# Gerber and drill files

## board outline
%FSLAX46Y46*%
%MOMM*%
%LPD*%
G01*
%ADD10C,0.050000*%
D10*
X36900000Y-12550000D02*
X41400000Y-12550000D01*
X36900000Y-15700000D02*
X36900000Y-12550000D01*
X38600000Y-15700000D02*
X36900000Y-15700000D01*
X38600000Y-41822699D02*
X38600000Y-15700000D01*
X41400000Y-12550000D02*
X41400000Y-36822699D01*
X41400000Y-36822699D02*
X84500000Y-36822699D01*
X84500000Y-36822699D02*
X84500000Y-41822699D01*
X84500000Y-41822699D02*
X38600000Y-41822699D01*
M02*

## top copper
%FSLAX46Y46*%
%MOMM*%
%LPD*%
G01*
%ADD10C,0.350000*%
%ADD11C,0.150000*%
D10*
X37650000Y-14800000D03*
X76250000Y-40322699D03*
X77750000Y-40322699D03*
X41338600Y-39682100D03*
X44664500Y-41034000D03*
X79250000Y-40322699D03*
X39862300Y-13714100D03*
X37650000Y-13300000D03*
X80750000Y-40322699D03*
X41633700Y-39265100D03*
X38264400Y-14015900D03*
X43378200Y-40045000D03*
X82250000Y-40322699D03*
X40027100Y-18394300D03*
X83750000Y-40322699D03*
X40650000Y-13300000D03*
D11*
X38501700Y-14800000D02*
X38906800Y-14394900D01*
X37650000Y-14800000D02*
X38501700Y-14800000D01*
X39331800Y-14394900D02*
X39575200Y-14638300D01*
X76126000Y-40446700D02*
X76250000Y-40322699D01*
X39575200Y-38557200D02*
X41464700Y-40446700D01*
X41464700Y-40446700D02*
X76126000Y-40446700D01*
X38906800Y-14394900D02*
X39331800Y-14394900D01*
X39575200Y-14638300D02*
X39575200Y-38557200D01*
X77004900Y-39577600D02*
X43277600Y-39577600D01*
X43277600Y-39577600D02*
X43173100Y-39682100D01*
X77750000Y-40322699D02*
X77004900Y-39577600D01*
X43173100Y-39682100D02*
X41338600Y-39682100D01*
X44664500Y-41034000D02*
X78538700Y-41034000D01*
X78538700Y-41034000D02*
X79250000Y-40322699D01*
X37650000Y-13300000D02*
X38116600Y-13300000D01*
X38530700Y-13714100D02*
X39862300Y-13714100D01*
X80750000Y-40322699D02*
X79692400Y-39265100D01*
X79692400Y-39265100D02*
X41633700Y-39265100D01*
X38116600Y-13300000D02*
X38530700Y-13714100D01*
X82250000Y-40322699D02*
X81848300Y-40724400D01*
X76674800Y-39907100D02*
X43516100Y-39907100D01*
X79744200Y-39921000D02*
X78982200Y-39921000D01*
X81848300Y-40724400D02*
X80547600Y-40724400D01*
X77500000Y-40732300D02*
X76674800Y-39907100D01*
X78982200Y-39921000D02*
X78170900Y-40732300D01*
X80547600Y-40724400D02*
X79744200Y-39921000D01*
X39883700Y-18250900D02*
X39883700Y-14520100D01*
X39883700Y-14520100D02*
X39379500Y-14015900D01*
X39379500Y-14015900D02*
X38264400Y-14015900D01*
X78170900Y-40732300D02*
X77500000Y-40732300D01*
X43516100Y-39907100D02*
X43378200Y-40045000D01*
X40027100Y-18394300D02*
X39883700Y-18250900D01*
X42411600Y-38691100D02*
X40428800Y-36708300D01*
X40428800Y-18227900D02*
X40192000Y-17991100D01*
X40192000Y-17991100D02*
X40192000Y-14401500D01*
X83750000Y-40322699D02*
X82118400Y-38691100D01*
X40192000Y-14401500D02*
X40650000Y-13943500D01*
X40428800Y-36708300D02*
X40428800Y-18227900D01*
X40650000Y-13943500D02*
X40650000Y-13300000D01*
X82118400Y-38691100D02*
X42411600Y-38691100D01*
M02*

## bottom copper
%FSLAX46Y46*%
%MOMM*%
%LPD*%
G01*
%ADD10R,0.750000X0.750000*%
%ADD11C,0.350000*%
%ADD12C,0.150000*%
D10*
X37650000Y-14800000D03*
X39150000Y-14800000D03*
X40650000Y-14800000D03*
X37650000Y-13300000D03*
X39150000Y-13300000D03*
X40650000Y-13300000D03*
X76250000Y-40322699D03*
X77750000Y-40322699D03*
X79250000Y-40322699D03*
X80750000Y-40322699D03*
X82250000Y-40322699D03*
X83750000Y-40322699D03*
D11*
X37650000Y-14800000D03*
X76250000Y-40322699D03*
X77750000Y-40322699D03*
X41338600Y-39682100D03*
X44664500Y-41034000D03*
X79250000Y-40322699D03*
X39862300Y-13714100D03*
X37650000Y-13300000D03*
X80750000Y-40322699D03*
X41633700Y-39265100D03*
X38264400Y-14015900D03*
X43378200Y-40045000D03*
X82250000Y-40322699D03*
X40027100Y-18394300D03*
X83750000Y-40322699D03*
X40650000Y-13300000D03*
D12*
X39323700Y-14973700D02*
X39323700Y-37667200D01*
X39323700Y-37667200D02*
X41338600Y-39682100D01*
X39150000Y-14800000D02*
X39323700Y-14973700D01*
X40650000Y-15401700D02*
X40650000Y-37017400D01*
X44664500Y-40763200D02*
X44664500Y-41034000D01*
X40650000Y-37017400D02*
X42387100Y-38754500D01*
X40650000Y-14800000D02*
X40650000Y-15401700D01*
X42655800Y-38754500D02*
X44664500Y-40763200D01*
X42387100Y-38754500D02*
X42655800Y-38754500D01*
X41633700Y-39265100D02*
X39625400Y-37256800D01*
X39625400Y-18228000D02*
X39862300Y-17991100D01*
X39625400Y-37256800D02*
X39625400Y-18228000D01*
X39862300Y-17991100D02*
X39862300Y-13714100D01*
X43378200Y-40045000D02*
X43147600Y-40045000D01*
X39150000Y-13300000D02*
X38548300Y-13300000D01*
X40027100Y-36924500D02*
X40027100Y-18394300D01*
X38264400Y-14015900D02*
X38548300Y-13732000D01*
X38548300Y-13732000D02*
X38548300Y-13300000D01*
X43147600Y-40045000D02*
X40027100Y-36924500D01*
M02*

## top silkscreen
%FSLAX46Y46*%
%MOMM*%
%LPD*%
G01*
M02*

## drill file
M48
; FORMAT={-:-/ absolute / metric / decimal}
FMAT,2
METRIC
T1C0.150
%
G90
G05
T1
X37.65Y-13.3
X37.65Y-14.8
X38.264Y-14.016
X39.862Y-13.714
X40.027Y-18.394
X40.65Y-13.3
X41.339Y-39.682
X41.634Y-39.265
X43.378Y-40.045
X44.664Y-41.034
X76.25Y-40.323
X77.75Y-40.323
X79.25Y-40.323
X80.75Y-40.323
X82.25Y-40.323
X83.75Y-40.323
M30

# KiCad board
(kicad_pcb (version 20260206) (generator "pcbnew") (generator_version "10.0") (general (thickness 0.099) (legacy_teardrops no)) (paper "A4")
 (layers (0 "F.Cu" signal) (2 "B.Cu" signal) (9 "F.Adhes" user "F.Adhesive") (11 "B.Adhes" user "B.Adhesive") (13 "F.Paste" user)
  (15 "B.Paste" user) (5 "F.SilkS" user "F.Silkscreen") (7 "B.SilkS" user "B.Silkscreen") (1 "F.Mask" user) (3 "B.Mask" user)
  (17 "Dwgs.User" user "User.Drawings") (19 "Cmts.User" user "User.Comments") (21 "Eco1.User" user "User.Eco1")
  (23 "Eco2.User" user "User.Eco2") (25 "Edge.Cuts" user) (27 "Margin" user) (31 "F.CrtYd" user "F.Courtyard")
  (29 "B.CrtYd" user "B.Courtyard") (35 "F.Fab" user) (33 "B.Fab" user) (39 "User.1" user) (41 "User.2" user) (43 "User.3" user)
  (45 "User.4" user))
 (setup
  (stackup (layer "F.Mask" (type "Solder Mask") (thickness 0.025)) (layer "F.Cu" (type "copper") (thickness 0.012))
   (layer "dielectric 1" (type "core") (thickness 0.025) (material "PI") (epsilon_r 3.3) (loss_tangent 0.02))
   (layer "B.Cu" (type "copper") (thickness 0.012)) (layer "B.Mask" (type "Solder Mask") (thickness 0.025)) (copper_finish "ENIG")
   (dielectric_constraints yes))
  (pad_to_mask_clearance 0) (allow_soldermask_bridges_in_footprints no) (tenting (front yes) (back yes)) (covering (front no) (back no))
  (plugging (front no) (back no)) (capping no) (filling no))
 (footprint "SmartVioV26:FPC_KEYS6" (layer "F.Cu") (at 0 0)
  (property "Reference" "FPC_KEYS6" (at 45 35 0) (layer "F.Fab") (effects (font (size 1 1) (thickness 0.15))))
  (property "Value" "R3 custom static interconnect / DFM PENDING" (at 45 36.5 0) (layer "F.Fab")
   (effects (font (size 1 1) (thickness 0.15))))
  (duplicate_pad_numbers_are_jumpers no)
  (pad "S1" smd rect (at 37.65 14.8) (size 0.75 0.75) (layers "B.Cu" "B.Mask") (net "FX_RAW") (solder_mask_margin 0.1))
  (pad "S2" smd rect (at 39.15 14.8) (size 0.75 0.75) (layers "B.Cu" "B.Mask") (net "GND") (solder_mask_margin 0.1))
  (pad "S3" smd rect (at 40.65 14.8) (size 0.75 0.75) (layers "B.Cu" "B.Mask") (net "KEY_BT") (solder_mask_margin 0.1))
  (pad "S4" smd rect (at 37.65 13.3) (size 0.75 0.75) (layers "B.Cu" "B.Mask") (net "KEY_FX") (solder_mask_margin 0.1))
  (pad "S5" smd rect (at 39.15 13.3) (size 0.75 0.75) (layers "B.Cu" "B.Mask") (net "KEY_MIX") (solder_mask_margin 0.1))
  (pad "S6" smd rect (at 40.65 13.3) (size 0.75 0.75) (layers "B.Cu" "B.Mask") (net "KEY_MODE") (solder_mask_margin 0.1))
  (pad "T1" smd rect (at 76.25 40.322699) (size 0.75 0.75) (layers "B.Cu" "B.Mask") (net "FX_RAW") (solder_mask_margin 0.1))
  (pad "T2" smd rect (at 77.75 40.322699) (size 0.75 0.75) (layers "B.Cu" "B.Mask") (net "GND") (solder_mask_margin 0.1))
  (pad "T3" smd rect (at 79.25 40.322699) (size 0.75 0.75) (layers "B.Cu" "B.Mask") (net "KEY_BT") (solder_mask_margin 0.1))
  (pad "T4" smd rect (at 80.75 40.322699) (size 0.75 0.75) (layers "B.Cu" "B.Mask") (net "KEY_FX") (solder_mask_margin 0.1))
  (pad "T5" smd rect (at 82.25 40.322699) (size 0.75 0.75) (layers "B.Cu" "B.Mask") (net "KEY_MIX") (solder_mask_margin 0.1))
  (pad "T6" smd rect (at 83.75 40.322699) (size 0.75 0.75) (layers "B.Cu" "B.Mask") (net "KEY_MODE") (solder_mask_margin 0.1)))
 (gr_line (start 36.9 12.55) (end 41.4 12.55) (stroke (width 0.05) (type default)) (layer "Edge.Cuts"))
 (gr_line (start 36.9 15.7) (end 36.9 12.55) (stroke (width 0.05) (type default)) (layer "Edge.Cuts"))
 (gr_line (start 38.6 15.7) (end 36.9 15.7) (stroke (width 0.05) (type default)) (layer "Edge.Cuts"))
 (gr_line (start 38.6 41.822699) (end 38.6 15.7) (stroke (width 0.05) (type default)) (layer "Edge.Cuts"))
 (gr_line (start 41.4 12.55) (end 41.4 36.822699) (stroke (width 0.05) (type default)) (layer "Edge.Cuts"))
 (gr_line (start 41.4 36.822699) (end 84.5 36.822699) (stroke (width 0.05) (type default)) (layer "Edge.Cuts"))
 (gr_line (start 84.5 36.822699) (end 84.5 41.822699) (stroke (width 0.05) (type default)) (layer "Edge.Cuts"))
 (gr_line (start 84.5 41.822699) (end 38.6 41.822699) (stroke (width 0.05) (type default)) (layer "Edge.Cuts"))
 (segment (start 38.5017 14.8) (end 38.9068 14.3949) (width 0.15) (layer "F.Cu") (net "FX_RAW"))
 (segment (start 37.65 14.8) (end 38.5017 14.8) (width 0.15) (layer "F.Cu") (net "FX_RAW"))
 (segment (start 39.3318 14.3949) (end 39.5752 14.6383) (width 0.15) (layer "F.Cu") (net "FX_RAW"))
 (segment (start 76.126 40.4467) (end 76.25 40.322699) (width 0.15) (layer "F.Cu") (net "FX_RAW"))
 (segment (start 39.5752 38.5572) (end 41.4647 40.4467) (width 0.15) (layer "F.Cu") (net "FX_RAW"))
 (segment (start 41.4647 40.4467) (end 76.126 40.4467) (width 0.15) (layer "F.Cu") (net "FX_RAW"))
 (segment (start 38.9068 14.3949) (end 39.3318 14.3949) (width 0.15) (layer "F.Cu") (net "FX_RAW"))
 (segment (start 39.5752 14.6383) (end 39.5752 38.5572) (width 0.15) (layer "F.Cu") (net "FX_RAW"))
 (via (at 37.65 14.8) (size 0.35) (drill 0.15) (layers "F.Cu" "B.Cu") (locked yes) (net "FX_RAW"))
 (via (at 76.25 40.322699) (size 0.35) (drill 0.15) (layers "F.Cu" "B.Cu") (locked yes) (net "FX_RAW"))
 (segment (start 77.0049 39.5776) (end 43.2776 39.5776) (width 0.15) (layer "F.Cu") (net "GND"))
 (segment (start 43.2776 39.5776) (end 43.1731 39.6821) (width 0.15) (layer "F.Cu") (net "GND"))
 (segment (start 77.75 40.322699) (end 77.0049 39.5776) (width 0.15) (layer "F.Cu") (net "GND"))
 (segment (start 43.1731 39.6821) (end 41.3386 39.6821) (width 0.15) (layer "F.Cu") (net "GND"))
 (via (at 77.75 40.322699) (size 0.35) (drill 0.15) (layers "F.Cu" "B.Cu") (locked yes) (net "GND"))
 (via (at 41.3386 39.6821) (size 0.35) (drill 0.15) (layers "F.Cu" "B.Cu") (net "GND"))
 (segment (start 39.3237 14.9737) (end 39.3237 37.6672) (width 0.15) (layer "B.Cu") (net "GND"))
 (segment (start 39.3237 37.6672) (end 41.3386 39.6821) (width 0.15) (layer "B.Cu") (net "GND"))
 (segment (start 39.15 14.8) (end 39.3237 14.9737) (width 0.15) (layer "B.Cu") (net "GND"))
 (segment (start 44.6645 41.034) (end 78.5387 41.034) (width 0.15) (layer "F.Cu") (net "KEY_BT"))
 (segment (start 78.5387 41.034) (end 79.25 40.322699) (width 0.15) (layer "F.Cu") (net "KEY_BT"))
 (via (at 44.6645 41.034) (size 0.35) (drill 0.15) (layers "F.Cu" "B.Cu") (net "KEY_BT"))
 (via (at 79.25 40.322699) (size 0.35) (drill 0.15) (layers "F.Cu" "B.Cu") (locked yes) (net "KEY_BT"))
 (segment (start 40.65 15.4017) (end 40.65 37.0174) (width 0.15) (layer "B.Cu") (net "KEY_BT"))
 (segment (start 44.6645 40.7632) (end 44.6645 41.034) (width 0.15) (layer "B.Cu") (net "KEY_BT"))
 (segment (start 40.65 37.0174) (end 42.3871 38.7545) (width 0.15) (layer "B.Cu") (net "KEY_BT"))
 (segment (start 40.65 14.8) (end 40.65 15.4017) (width 0.15) (layer "B.Cu") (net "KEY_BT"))
 (segment (start 42.6558 38.7545) (end 44.6645 40.7632) (width 0.15) (layer "B.Cu") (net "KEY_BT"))
 (segment (start 42.3871 38.7545) (end 42.6558 38.7545) (width 0.15) (layer "B.Cu") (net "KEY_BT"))
 (segment (start 37.65 13.3) (end 38.1166 13.3) (width 0.15) (layer "F.Cu") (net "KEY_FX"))
 (segment (start 38.5307 13.7141) (end 39.8623 13.7141) (width 0.15) (layer "F.Cu") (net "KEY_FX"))
 (segment (start 80.75 40.322699) (end 79.6924 39.2651) (width 0.15) (layer "F.Cu") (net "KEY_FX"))
 (segment (start 79.6924 39.2651) (end 41.6337 39.2651) (width 0.15) (layer "F.Cu") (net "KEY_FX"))
 (segment (start 38.1166 13.3) (end 38.5307 13.7141) (width 0.15) (layer "F.Cu") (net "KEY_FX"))
 (via (at 39.8623 13.7141) (size 0.35) (drill 0.15) (layers "F.Cu" "B.Cu") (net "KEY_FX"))
 (via (at 37.65 13.3) (size 0.35) (drill 0.15) (layers "F.Cu" "B.Cu") (locked yes) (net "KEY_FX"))
 (via (at 80.75 40.322699) (size 0.35) (drill 0.15) (layers "F.Cu" "B.Cu") (locked yes) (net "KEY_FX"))
 (via (at 41.6337 39.2651) (size 0.35) (drill 0.15) (layers "F.Cu" "B.Cu") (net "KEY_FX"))
 (segment (start 41.6337 39.2651) (end 39.6254 37.2568) (width 0.15) (layer "B.Cu") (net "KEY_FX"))
 (segment (start 39.6254 18.228) (end 39.8623 17.9911) (width 0.15) (layer "B.Cu") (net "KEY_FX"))
 (segment (start 39.6254 37.2568) (end 39.6254 18.228) (width 0.15) (layer "B.Cu") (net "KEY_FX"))
 (segment (start 39.8623 17.9911) (end 39.8623 13.7141) (width 0.15) (layer "B.Cu") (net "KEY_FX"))
 (segment (start 82.25 40.322699) (end 81.8483 40.7244) (width 0.15) (layer "F.Cu") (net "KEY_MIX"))
 (segment (start 76.6748 39.9071) (end 43.5161 39.9071) (width 0.15) (layer "F.Cu") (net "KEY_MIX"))
 (segment (start 79.7442 39.921) (end 78.9822 39.921) (width 0.15) (layer "F.Cu") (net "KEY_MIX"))
 (segment (start 81.8483 40.7244) (end 80.5476 40.7244) (width 0.15) (layer "F.Cu") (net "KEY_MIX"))
 (segment (start 77.5 40.7323) (end 76.6748 39.9071) (width 0.15) (layer "F.Cu") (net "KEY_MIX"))
 (segment (start 78.9822 39.921) (end 78.1709 40.7323) (width 0.15) (layer "F.Cu") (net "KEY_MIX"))
 (segment (start 80.5476 40.7244) (end 79.7442 39.921) (width 0.15) (layer "F.Cu") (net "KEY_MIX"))
 (segment (start 39.8837 18.2509) (end 39.8837 14.5201) (width 0.15) (layer "F.Cu") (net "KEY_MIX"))
 (segment (start 39.8837 14.5201) (end 39.3795 14.0159) (width 0.15) (layer "F.Cu") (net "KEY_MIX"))
 (segment (start 39.3795 14.0159) (end 38.2644 14.0159) (width 0.15) (layer "F.Cu") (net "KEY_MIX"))
 (segment (start 78.1709 40.7323) (end 77.5 40.7323) (width 0.15) (layer "F.Cu") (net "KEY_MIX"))
 (segment (start 43.5161 39.9071) (end 43.3782 40.045) (width 0.15) (layer "F.Cu") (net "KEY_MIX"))
 (segment (start 40.0271 18.3943) (end 39.8837 18.2509) (width 0.15) (layer "F.Cu") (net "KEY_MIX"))
 (via (at 38.2644 14.0159) (size 0.35) (drill 0.15) (layers "F.Cu" "B.Cu") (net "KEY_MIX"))
 (via (at 43.3782 40.045) (size 0.35) (drill 0.15) (layers "F.Cu" "B.Cu") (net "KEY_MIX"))
 (via (at 82.25 40.322699) (size 0.35) (drill 0.15) (layers "F.Cu" "B.Cu") (locked yes) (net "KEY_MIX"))
 (via (at 40.0271 18.3943) (size 0.35) (drill 0.15) (layers "F.Cu" "B.Cu") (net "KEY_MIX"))
 (segment (start 43.3782 40.045) (end 43.1476 40.045) (width 0.15) (layer "B.Cu") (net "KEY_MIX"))
 (segment (start 39.15 13.3) (end 38.5483 13.3) (width 0.15) (layer "B.Cu") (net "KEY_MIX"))
 (segment (start 40.0271 36.9245) (end 40.0271 18.3943) (width 0.15) (layer "B.Cu") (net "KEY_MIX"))
 (segment (start 38.2644 14.0159) (end 38.5483 13.732) (width 0.15) (layer "B.Cu") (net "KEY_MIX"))
 (segment (start 38.5483 13.732) (end 38.5483 13.3) (width 0.15) (layer "B.Cu") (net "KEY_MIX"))
 (segment (start 43.1476 40.045) (end 40.0271 36.9245) (width 0.15) (layer "B.Cu") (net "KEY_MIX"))
 (segment (start 42.4116 38.6911) (end 40.4288 36.7083) (width 0.15) (layer "F.Cu") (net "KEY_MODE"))
 (segment (start 40.4288 18.2279) (end 40.192 17.9911) (width 0.15) (layer "F.Cu") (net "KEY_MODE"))
 (segment (start 40.192 17.9911) (end 40.192 14.4015) (width 0.15) (layer "F.Cu") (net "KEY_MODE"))
 (segment (start 83.75 40.322699) (end 82.1184 38.6911) (width 0.15) (layer "F.Cu") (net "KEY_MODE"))
 (segment (start 40.192 14.4015) (end 40.65 13.9435) (width 0.15) (layer "F.Cu") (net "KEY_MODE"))
 (segment (start 40.4288 36.7083) (end 40.4288 18.2279) (width 0.15) (layer "F.Cu") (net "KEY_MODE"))
 (segment (start 40.65 13.9435) (end 40.65 13.3) (width 0.15) (layer "F.Cu") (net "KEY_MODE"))
 (segment (start 82.1184 38.6911) (end 42.4116 38.6911) (width 0.15) (layer "F.Cu") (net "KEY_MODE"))
 (via (at 83.75 40.322699) (size 0.35) (drill 0.15) (layers "F.Cu" "B.Cu") (locked yes) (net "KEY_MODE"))
 (via (at 40.65 13.3) (size 0.35) (drill 0.15) (layers "F.Cu" "B.Cu") (locked yes) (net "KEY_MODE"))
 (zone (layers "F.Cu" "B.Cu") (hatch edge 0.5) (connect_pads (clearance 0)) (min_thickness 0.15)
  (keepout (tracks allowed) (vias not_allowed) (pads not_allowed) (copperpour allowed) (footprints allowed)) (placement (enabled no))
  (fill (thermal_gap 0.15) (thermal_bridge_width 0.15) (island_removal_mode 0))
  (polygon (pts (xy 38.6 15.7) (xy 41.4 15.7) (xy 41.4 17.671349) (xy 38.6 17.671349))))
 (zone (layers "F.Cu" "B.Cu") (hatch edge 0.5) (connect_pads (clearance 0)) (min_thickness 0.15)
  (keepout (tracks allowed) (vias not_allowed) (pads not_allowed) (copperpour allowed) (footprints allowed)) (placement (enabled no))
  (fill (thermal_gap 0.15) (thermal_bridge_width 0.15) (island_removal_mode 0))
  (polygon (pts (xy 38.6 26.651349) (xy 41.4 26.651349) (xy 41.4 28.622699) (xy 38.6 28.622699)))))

